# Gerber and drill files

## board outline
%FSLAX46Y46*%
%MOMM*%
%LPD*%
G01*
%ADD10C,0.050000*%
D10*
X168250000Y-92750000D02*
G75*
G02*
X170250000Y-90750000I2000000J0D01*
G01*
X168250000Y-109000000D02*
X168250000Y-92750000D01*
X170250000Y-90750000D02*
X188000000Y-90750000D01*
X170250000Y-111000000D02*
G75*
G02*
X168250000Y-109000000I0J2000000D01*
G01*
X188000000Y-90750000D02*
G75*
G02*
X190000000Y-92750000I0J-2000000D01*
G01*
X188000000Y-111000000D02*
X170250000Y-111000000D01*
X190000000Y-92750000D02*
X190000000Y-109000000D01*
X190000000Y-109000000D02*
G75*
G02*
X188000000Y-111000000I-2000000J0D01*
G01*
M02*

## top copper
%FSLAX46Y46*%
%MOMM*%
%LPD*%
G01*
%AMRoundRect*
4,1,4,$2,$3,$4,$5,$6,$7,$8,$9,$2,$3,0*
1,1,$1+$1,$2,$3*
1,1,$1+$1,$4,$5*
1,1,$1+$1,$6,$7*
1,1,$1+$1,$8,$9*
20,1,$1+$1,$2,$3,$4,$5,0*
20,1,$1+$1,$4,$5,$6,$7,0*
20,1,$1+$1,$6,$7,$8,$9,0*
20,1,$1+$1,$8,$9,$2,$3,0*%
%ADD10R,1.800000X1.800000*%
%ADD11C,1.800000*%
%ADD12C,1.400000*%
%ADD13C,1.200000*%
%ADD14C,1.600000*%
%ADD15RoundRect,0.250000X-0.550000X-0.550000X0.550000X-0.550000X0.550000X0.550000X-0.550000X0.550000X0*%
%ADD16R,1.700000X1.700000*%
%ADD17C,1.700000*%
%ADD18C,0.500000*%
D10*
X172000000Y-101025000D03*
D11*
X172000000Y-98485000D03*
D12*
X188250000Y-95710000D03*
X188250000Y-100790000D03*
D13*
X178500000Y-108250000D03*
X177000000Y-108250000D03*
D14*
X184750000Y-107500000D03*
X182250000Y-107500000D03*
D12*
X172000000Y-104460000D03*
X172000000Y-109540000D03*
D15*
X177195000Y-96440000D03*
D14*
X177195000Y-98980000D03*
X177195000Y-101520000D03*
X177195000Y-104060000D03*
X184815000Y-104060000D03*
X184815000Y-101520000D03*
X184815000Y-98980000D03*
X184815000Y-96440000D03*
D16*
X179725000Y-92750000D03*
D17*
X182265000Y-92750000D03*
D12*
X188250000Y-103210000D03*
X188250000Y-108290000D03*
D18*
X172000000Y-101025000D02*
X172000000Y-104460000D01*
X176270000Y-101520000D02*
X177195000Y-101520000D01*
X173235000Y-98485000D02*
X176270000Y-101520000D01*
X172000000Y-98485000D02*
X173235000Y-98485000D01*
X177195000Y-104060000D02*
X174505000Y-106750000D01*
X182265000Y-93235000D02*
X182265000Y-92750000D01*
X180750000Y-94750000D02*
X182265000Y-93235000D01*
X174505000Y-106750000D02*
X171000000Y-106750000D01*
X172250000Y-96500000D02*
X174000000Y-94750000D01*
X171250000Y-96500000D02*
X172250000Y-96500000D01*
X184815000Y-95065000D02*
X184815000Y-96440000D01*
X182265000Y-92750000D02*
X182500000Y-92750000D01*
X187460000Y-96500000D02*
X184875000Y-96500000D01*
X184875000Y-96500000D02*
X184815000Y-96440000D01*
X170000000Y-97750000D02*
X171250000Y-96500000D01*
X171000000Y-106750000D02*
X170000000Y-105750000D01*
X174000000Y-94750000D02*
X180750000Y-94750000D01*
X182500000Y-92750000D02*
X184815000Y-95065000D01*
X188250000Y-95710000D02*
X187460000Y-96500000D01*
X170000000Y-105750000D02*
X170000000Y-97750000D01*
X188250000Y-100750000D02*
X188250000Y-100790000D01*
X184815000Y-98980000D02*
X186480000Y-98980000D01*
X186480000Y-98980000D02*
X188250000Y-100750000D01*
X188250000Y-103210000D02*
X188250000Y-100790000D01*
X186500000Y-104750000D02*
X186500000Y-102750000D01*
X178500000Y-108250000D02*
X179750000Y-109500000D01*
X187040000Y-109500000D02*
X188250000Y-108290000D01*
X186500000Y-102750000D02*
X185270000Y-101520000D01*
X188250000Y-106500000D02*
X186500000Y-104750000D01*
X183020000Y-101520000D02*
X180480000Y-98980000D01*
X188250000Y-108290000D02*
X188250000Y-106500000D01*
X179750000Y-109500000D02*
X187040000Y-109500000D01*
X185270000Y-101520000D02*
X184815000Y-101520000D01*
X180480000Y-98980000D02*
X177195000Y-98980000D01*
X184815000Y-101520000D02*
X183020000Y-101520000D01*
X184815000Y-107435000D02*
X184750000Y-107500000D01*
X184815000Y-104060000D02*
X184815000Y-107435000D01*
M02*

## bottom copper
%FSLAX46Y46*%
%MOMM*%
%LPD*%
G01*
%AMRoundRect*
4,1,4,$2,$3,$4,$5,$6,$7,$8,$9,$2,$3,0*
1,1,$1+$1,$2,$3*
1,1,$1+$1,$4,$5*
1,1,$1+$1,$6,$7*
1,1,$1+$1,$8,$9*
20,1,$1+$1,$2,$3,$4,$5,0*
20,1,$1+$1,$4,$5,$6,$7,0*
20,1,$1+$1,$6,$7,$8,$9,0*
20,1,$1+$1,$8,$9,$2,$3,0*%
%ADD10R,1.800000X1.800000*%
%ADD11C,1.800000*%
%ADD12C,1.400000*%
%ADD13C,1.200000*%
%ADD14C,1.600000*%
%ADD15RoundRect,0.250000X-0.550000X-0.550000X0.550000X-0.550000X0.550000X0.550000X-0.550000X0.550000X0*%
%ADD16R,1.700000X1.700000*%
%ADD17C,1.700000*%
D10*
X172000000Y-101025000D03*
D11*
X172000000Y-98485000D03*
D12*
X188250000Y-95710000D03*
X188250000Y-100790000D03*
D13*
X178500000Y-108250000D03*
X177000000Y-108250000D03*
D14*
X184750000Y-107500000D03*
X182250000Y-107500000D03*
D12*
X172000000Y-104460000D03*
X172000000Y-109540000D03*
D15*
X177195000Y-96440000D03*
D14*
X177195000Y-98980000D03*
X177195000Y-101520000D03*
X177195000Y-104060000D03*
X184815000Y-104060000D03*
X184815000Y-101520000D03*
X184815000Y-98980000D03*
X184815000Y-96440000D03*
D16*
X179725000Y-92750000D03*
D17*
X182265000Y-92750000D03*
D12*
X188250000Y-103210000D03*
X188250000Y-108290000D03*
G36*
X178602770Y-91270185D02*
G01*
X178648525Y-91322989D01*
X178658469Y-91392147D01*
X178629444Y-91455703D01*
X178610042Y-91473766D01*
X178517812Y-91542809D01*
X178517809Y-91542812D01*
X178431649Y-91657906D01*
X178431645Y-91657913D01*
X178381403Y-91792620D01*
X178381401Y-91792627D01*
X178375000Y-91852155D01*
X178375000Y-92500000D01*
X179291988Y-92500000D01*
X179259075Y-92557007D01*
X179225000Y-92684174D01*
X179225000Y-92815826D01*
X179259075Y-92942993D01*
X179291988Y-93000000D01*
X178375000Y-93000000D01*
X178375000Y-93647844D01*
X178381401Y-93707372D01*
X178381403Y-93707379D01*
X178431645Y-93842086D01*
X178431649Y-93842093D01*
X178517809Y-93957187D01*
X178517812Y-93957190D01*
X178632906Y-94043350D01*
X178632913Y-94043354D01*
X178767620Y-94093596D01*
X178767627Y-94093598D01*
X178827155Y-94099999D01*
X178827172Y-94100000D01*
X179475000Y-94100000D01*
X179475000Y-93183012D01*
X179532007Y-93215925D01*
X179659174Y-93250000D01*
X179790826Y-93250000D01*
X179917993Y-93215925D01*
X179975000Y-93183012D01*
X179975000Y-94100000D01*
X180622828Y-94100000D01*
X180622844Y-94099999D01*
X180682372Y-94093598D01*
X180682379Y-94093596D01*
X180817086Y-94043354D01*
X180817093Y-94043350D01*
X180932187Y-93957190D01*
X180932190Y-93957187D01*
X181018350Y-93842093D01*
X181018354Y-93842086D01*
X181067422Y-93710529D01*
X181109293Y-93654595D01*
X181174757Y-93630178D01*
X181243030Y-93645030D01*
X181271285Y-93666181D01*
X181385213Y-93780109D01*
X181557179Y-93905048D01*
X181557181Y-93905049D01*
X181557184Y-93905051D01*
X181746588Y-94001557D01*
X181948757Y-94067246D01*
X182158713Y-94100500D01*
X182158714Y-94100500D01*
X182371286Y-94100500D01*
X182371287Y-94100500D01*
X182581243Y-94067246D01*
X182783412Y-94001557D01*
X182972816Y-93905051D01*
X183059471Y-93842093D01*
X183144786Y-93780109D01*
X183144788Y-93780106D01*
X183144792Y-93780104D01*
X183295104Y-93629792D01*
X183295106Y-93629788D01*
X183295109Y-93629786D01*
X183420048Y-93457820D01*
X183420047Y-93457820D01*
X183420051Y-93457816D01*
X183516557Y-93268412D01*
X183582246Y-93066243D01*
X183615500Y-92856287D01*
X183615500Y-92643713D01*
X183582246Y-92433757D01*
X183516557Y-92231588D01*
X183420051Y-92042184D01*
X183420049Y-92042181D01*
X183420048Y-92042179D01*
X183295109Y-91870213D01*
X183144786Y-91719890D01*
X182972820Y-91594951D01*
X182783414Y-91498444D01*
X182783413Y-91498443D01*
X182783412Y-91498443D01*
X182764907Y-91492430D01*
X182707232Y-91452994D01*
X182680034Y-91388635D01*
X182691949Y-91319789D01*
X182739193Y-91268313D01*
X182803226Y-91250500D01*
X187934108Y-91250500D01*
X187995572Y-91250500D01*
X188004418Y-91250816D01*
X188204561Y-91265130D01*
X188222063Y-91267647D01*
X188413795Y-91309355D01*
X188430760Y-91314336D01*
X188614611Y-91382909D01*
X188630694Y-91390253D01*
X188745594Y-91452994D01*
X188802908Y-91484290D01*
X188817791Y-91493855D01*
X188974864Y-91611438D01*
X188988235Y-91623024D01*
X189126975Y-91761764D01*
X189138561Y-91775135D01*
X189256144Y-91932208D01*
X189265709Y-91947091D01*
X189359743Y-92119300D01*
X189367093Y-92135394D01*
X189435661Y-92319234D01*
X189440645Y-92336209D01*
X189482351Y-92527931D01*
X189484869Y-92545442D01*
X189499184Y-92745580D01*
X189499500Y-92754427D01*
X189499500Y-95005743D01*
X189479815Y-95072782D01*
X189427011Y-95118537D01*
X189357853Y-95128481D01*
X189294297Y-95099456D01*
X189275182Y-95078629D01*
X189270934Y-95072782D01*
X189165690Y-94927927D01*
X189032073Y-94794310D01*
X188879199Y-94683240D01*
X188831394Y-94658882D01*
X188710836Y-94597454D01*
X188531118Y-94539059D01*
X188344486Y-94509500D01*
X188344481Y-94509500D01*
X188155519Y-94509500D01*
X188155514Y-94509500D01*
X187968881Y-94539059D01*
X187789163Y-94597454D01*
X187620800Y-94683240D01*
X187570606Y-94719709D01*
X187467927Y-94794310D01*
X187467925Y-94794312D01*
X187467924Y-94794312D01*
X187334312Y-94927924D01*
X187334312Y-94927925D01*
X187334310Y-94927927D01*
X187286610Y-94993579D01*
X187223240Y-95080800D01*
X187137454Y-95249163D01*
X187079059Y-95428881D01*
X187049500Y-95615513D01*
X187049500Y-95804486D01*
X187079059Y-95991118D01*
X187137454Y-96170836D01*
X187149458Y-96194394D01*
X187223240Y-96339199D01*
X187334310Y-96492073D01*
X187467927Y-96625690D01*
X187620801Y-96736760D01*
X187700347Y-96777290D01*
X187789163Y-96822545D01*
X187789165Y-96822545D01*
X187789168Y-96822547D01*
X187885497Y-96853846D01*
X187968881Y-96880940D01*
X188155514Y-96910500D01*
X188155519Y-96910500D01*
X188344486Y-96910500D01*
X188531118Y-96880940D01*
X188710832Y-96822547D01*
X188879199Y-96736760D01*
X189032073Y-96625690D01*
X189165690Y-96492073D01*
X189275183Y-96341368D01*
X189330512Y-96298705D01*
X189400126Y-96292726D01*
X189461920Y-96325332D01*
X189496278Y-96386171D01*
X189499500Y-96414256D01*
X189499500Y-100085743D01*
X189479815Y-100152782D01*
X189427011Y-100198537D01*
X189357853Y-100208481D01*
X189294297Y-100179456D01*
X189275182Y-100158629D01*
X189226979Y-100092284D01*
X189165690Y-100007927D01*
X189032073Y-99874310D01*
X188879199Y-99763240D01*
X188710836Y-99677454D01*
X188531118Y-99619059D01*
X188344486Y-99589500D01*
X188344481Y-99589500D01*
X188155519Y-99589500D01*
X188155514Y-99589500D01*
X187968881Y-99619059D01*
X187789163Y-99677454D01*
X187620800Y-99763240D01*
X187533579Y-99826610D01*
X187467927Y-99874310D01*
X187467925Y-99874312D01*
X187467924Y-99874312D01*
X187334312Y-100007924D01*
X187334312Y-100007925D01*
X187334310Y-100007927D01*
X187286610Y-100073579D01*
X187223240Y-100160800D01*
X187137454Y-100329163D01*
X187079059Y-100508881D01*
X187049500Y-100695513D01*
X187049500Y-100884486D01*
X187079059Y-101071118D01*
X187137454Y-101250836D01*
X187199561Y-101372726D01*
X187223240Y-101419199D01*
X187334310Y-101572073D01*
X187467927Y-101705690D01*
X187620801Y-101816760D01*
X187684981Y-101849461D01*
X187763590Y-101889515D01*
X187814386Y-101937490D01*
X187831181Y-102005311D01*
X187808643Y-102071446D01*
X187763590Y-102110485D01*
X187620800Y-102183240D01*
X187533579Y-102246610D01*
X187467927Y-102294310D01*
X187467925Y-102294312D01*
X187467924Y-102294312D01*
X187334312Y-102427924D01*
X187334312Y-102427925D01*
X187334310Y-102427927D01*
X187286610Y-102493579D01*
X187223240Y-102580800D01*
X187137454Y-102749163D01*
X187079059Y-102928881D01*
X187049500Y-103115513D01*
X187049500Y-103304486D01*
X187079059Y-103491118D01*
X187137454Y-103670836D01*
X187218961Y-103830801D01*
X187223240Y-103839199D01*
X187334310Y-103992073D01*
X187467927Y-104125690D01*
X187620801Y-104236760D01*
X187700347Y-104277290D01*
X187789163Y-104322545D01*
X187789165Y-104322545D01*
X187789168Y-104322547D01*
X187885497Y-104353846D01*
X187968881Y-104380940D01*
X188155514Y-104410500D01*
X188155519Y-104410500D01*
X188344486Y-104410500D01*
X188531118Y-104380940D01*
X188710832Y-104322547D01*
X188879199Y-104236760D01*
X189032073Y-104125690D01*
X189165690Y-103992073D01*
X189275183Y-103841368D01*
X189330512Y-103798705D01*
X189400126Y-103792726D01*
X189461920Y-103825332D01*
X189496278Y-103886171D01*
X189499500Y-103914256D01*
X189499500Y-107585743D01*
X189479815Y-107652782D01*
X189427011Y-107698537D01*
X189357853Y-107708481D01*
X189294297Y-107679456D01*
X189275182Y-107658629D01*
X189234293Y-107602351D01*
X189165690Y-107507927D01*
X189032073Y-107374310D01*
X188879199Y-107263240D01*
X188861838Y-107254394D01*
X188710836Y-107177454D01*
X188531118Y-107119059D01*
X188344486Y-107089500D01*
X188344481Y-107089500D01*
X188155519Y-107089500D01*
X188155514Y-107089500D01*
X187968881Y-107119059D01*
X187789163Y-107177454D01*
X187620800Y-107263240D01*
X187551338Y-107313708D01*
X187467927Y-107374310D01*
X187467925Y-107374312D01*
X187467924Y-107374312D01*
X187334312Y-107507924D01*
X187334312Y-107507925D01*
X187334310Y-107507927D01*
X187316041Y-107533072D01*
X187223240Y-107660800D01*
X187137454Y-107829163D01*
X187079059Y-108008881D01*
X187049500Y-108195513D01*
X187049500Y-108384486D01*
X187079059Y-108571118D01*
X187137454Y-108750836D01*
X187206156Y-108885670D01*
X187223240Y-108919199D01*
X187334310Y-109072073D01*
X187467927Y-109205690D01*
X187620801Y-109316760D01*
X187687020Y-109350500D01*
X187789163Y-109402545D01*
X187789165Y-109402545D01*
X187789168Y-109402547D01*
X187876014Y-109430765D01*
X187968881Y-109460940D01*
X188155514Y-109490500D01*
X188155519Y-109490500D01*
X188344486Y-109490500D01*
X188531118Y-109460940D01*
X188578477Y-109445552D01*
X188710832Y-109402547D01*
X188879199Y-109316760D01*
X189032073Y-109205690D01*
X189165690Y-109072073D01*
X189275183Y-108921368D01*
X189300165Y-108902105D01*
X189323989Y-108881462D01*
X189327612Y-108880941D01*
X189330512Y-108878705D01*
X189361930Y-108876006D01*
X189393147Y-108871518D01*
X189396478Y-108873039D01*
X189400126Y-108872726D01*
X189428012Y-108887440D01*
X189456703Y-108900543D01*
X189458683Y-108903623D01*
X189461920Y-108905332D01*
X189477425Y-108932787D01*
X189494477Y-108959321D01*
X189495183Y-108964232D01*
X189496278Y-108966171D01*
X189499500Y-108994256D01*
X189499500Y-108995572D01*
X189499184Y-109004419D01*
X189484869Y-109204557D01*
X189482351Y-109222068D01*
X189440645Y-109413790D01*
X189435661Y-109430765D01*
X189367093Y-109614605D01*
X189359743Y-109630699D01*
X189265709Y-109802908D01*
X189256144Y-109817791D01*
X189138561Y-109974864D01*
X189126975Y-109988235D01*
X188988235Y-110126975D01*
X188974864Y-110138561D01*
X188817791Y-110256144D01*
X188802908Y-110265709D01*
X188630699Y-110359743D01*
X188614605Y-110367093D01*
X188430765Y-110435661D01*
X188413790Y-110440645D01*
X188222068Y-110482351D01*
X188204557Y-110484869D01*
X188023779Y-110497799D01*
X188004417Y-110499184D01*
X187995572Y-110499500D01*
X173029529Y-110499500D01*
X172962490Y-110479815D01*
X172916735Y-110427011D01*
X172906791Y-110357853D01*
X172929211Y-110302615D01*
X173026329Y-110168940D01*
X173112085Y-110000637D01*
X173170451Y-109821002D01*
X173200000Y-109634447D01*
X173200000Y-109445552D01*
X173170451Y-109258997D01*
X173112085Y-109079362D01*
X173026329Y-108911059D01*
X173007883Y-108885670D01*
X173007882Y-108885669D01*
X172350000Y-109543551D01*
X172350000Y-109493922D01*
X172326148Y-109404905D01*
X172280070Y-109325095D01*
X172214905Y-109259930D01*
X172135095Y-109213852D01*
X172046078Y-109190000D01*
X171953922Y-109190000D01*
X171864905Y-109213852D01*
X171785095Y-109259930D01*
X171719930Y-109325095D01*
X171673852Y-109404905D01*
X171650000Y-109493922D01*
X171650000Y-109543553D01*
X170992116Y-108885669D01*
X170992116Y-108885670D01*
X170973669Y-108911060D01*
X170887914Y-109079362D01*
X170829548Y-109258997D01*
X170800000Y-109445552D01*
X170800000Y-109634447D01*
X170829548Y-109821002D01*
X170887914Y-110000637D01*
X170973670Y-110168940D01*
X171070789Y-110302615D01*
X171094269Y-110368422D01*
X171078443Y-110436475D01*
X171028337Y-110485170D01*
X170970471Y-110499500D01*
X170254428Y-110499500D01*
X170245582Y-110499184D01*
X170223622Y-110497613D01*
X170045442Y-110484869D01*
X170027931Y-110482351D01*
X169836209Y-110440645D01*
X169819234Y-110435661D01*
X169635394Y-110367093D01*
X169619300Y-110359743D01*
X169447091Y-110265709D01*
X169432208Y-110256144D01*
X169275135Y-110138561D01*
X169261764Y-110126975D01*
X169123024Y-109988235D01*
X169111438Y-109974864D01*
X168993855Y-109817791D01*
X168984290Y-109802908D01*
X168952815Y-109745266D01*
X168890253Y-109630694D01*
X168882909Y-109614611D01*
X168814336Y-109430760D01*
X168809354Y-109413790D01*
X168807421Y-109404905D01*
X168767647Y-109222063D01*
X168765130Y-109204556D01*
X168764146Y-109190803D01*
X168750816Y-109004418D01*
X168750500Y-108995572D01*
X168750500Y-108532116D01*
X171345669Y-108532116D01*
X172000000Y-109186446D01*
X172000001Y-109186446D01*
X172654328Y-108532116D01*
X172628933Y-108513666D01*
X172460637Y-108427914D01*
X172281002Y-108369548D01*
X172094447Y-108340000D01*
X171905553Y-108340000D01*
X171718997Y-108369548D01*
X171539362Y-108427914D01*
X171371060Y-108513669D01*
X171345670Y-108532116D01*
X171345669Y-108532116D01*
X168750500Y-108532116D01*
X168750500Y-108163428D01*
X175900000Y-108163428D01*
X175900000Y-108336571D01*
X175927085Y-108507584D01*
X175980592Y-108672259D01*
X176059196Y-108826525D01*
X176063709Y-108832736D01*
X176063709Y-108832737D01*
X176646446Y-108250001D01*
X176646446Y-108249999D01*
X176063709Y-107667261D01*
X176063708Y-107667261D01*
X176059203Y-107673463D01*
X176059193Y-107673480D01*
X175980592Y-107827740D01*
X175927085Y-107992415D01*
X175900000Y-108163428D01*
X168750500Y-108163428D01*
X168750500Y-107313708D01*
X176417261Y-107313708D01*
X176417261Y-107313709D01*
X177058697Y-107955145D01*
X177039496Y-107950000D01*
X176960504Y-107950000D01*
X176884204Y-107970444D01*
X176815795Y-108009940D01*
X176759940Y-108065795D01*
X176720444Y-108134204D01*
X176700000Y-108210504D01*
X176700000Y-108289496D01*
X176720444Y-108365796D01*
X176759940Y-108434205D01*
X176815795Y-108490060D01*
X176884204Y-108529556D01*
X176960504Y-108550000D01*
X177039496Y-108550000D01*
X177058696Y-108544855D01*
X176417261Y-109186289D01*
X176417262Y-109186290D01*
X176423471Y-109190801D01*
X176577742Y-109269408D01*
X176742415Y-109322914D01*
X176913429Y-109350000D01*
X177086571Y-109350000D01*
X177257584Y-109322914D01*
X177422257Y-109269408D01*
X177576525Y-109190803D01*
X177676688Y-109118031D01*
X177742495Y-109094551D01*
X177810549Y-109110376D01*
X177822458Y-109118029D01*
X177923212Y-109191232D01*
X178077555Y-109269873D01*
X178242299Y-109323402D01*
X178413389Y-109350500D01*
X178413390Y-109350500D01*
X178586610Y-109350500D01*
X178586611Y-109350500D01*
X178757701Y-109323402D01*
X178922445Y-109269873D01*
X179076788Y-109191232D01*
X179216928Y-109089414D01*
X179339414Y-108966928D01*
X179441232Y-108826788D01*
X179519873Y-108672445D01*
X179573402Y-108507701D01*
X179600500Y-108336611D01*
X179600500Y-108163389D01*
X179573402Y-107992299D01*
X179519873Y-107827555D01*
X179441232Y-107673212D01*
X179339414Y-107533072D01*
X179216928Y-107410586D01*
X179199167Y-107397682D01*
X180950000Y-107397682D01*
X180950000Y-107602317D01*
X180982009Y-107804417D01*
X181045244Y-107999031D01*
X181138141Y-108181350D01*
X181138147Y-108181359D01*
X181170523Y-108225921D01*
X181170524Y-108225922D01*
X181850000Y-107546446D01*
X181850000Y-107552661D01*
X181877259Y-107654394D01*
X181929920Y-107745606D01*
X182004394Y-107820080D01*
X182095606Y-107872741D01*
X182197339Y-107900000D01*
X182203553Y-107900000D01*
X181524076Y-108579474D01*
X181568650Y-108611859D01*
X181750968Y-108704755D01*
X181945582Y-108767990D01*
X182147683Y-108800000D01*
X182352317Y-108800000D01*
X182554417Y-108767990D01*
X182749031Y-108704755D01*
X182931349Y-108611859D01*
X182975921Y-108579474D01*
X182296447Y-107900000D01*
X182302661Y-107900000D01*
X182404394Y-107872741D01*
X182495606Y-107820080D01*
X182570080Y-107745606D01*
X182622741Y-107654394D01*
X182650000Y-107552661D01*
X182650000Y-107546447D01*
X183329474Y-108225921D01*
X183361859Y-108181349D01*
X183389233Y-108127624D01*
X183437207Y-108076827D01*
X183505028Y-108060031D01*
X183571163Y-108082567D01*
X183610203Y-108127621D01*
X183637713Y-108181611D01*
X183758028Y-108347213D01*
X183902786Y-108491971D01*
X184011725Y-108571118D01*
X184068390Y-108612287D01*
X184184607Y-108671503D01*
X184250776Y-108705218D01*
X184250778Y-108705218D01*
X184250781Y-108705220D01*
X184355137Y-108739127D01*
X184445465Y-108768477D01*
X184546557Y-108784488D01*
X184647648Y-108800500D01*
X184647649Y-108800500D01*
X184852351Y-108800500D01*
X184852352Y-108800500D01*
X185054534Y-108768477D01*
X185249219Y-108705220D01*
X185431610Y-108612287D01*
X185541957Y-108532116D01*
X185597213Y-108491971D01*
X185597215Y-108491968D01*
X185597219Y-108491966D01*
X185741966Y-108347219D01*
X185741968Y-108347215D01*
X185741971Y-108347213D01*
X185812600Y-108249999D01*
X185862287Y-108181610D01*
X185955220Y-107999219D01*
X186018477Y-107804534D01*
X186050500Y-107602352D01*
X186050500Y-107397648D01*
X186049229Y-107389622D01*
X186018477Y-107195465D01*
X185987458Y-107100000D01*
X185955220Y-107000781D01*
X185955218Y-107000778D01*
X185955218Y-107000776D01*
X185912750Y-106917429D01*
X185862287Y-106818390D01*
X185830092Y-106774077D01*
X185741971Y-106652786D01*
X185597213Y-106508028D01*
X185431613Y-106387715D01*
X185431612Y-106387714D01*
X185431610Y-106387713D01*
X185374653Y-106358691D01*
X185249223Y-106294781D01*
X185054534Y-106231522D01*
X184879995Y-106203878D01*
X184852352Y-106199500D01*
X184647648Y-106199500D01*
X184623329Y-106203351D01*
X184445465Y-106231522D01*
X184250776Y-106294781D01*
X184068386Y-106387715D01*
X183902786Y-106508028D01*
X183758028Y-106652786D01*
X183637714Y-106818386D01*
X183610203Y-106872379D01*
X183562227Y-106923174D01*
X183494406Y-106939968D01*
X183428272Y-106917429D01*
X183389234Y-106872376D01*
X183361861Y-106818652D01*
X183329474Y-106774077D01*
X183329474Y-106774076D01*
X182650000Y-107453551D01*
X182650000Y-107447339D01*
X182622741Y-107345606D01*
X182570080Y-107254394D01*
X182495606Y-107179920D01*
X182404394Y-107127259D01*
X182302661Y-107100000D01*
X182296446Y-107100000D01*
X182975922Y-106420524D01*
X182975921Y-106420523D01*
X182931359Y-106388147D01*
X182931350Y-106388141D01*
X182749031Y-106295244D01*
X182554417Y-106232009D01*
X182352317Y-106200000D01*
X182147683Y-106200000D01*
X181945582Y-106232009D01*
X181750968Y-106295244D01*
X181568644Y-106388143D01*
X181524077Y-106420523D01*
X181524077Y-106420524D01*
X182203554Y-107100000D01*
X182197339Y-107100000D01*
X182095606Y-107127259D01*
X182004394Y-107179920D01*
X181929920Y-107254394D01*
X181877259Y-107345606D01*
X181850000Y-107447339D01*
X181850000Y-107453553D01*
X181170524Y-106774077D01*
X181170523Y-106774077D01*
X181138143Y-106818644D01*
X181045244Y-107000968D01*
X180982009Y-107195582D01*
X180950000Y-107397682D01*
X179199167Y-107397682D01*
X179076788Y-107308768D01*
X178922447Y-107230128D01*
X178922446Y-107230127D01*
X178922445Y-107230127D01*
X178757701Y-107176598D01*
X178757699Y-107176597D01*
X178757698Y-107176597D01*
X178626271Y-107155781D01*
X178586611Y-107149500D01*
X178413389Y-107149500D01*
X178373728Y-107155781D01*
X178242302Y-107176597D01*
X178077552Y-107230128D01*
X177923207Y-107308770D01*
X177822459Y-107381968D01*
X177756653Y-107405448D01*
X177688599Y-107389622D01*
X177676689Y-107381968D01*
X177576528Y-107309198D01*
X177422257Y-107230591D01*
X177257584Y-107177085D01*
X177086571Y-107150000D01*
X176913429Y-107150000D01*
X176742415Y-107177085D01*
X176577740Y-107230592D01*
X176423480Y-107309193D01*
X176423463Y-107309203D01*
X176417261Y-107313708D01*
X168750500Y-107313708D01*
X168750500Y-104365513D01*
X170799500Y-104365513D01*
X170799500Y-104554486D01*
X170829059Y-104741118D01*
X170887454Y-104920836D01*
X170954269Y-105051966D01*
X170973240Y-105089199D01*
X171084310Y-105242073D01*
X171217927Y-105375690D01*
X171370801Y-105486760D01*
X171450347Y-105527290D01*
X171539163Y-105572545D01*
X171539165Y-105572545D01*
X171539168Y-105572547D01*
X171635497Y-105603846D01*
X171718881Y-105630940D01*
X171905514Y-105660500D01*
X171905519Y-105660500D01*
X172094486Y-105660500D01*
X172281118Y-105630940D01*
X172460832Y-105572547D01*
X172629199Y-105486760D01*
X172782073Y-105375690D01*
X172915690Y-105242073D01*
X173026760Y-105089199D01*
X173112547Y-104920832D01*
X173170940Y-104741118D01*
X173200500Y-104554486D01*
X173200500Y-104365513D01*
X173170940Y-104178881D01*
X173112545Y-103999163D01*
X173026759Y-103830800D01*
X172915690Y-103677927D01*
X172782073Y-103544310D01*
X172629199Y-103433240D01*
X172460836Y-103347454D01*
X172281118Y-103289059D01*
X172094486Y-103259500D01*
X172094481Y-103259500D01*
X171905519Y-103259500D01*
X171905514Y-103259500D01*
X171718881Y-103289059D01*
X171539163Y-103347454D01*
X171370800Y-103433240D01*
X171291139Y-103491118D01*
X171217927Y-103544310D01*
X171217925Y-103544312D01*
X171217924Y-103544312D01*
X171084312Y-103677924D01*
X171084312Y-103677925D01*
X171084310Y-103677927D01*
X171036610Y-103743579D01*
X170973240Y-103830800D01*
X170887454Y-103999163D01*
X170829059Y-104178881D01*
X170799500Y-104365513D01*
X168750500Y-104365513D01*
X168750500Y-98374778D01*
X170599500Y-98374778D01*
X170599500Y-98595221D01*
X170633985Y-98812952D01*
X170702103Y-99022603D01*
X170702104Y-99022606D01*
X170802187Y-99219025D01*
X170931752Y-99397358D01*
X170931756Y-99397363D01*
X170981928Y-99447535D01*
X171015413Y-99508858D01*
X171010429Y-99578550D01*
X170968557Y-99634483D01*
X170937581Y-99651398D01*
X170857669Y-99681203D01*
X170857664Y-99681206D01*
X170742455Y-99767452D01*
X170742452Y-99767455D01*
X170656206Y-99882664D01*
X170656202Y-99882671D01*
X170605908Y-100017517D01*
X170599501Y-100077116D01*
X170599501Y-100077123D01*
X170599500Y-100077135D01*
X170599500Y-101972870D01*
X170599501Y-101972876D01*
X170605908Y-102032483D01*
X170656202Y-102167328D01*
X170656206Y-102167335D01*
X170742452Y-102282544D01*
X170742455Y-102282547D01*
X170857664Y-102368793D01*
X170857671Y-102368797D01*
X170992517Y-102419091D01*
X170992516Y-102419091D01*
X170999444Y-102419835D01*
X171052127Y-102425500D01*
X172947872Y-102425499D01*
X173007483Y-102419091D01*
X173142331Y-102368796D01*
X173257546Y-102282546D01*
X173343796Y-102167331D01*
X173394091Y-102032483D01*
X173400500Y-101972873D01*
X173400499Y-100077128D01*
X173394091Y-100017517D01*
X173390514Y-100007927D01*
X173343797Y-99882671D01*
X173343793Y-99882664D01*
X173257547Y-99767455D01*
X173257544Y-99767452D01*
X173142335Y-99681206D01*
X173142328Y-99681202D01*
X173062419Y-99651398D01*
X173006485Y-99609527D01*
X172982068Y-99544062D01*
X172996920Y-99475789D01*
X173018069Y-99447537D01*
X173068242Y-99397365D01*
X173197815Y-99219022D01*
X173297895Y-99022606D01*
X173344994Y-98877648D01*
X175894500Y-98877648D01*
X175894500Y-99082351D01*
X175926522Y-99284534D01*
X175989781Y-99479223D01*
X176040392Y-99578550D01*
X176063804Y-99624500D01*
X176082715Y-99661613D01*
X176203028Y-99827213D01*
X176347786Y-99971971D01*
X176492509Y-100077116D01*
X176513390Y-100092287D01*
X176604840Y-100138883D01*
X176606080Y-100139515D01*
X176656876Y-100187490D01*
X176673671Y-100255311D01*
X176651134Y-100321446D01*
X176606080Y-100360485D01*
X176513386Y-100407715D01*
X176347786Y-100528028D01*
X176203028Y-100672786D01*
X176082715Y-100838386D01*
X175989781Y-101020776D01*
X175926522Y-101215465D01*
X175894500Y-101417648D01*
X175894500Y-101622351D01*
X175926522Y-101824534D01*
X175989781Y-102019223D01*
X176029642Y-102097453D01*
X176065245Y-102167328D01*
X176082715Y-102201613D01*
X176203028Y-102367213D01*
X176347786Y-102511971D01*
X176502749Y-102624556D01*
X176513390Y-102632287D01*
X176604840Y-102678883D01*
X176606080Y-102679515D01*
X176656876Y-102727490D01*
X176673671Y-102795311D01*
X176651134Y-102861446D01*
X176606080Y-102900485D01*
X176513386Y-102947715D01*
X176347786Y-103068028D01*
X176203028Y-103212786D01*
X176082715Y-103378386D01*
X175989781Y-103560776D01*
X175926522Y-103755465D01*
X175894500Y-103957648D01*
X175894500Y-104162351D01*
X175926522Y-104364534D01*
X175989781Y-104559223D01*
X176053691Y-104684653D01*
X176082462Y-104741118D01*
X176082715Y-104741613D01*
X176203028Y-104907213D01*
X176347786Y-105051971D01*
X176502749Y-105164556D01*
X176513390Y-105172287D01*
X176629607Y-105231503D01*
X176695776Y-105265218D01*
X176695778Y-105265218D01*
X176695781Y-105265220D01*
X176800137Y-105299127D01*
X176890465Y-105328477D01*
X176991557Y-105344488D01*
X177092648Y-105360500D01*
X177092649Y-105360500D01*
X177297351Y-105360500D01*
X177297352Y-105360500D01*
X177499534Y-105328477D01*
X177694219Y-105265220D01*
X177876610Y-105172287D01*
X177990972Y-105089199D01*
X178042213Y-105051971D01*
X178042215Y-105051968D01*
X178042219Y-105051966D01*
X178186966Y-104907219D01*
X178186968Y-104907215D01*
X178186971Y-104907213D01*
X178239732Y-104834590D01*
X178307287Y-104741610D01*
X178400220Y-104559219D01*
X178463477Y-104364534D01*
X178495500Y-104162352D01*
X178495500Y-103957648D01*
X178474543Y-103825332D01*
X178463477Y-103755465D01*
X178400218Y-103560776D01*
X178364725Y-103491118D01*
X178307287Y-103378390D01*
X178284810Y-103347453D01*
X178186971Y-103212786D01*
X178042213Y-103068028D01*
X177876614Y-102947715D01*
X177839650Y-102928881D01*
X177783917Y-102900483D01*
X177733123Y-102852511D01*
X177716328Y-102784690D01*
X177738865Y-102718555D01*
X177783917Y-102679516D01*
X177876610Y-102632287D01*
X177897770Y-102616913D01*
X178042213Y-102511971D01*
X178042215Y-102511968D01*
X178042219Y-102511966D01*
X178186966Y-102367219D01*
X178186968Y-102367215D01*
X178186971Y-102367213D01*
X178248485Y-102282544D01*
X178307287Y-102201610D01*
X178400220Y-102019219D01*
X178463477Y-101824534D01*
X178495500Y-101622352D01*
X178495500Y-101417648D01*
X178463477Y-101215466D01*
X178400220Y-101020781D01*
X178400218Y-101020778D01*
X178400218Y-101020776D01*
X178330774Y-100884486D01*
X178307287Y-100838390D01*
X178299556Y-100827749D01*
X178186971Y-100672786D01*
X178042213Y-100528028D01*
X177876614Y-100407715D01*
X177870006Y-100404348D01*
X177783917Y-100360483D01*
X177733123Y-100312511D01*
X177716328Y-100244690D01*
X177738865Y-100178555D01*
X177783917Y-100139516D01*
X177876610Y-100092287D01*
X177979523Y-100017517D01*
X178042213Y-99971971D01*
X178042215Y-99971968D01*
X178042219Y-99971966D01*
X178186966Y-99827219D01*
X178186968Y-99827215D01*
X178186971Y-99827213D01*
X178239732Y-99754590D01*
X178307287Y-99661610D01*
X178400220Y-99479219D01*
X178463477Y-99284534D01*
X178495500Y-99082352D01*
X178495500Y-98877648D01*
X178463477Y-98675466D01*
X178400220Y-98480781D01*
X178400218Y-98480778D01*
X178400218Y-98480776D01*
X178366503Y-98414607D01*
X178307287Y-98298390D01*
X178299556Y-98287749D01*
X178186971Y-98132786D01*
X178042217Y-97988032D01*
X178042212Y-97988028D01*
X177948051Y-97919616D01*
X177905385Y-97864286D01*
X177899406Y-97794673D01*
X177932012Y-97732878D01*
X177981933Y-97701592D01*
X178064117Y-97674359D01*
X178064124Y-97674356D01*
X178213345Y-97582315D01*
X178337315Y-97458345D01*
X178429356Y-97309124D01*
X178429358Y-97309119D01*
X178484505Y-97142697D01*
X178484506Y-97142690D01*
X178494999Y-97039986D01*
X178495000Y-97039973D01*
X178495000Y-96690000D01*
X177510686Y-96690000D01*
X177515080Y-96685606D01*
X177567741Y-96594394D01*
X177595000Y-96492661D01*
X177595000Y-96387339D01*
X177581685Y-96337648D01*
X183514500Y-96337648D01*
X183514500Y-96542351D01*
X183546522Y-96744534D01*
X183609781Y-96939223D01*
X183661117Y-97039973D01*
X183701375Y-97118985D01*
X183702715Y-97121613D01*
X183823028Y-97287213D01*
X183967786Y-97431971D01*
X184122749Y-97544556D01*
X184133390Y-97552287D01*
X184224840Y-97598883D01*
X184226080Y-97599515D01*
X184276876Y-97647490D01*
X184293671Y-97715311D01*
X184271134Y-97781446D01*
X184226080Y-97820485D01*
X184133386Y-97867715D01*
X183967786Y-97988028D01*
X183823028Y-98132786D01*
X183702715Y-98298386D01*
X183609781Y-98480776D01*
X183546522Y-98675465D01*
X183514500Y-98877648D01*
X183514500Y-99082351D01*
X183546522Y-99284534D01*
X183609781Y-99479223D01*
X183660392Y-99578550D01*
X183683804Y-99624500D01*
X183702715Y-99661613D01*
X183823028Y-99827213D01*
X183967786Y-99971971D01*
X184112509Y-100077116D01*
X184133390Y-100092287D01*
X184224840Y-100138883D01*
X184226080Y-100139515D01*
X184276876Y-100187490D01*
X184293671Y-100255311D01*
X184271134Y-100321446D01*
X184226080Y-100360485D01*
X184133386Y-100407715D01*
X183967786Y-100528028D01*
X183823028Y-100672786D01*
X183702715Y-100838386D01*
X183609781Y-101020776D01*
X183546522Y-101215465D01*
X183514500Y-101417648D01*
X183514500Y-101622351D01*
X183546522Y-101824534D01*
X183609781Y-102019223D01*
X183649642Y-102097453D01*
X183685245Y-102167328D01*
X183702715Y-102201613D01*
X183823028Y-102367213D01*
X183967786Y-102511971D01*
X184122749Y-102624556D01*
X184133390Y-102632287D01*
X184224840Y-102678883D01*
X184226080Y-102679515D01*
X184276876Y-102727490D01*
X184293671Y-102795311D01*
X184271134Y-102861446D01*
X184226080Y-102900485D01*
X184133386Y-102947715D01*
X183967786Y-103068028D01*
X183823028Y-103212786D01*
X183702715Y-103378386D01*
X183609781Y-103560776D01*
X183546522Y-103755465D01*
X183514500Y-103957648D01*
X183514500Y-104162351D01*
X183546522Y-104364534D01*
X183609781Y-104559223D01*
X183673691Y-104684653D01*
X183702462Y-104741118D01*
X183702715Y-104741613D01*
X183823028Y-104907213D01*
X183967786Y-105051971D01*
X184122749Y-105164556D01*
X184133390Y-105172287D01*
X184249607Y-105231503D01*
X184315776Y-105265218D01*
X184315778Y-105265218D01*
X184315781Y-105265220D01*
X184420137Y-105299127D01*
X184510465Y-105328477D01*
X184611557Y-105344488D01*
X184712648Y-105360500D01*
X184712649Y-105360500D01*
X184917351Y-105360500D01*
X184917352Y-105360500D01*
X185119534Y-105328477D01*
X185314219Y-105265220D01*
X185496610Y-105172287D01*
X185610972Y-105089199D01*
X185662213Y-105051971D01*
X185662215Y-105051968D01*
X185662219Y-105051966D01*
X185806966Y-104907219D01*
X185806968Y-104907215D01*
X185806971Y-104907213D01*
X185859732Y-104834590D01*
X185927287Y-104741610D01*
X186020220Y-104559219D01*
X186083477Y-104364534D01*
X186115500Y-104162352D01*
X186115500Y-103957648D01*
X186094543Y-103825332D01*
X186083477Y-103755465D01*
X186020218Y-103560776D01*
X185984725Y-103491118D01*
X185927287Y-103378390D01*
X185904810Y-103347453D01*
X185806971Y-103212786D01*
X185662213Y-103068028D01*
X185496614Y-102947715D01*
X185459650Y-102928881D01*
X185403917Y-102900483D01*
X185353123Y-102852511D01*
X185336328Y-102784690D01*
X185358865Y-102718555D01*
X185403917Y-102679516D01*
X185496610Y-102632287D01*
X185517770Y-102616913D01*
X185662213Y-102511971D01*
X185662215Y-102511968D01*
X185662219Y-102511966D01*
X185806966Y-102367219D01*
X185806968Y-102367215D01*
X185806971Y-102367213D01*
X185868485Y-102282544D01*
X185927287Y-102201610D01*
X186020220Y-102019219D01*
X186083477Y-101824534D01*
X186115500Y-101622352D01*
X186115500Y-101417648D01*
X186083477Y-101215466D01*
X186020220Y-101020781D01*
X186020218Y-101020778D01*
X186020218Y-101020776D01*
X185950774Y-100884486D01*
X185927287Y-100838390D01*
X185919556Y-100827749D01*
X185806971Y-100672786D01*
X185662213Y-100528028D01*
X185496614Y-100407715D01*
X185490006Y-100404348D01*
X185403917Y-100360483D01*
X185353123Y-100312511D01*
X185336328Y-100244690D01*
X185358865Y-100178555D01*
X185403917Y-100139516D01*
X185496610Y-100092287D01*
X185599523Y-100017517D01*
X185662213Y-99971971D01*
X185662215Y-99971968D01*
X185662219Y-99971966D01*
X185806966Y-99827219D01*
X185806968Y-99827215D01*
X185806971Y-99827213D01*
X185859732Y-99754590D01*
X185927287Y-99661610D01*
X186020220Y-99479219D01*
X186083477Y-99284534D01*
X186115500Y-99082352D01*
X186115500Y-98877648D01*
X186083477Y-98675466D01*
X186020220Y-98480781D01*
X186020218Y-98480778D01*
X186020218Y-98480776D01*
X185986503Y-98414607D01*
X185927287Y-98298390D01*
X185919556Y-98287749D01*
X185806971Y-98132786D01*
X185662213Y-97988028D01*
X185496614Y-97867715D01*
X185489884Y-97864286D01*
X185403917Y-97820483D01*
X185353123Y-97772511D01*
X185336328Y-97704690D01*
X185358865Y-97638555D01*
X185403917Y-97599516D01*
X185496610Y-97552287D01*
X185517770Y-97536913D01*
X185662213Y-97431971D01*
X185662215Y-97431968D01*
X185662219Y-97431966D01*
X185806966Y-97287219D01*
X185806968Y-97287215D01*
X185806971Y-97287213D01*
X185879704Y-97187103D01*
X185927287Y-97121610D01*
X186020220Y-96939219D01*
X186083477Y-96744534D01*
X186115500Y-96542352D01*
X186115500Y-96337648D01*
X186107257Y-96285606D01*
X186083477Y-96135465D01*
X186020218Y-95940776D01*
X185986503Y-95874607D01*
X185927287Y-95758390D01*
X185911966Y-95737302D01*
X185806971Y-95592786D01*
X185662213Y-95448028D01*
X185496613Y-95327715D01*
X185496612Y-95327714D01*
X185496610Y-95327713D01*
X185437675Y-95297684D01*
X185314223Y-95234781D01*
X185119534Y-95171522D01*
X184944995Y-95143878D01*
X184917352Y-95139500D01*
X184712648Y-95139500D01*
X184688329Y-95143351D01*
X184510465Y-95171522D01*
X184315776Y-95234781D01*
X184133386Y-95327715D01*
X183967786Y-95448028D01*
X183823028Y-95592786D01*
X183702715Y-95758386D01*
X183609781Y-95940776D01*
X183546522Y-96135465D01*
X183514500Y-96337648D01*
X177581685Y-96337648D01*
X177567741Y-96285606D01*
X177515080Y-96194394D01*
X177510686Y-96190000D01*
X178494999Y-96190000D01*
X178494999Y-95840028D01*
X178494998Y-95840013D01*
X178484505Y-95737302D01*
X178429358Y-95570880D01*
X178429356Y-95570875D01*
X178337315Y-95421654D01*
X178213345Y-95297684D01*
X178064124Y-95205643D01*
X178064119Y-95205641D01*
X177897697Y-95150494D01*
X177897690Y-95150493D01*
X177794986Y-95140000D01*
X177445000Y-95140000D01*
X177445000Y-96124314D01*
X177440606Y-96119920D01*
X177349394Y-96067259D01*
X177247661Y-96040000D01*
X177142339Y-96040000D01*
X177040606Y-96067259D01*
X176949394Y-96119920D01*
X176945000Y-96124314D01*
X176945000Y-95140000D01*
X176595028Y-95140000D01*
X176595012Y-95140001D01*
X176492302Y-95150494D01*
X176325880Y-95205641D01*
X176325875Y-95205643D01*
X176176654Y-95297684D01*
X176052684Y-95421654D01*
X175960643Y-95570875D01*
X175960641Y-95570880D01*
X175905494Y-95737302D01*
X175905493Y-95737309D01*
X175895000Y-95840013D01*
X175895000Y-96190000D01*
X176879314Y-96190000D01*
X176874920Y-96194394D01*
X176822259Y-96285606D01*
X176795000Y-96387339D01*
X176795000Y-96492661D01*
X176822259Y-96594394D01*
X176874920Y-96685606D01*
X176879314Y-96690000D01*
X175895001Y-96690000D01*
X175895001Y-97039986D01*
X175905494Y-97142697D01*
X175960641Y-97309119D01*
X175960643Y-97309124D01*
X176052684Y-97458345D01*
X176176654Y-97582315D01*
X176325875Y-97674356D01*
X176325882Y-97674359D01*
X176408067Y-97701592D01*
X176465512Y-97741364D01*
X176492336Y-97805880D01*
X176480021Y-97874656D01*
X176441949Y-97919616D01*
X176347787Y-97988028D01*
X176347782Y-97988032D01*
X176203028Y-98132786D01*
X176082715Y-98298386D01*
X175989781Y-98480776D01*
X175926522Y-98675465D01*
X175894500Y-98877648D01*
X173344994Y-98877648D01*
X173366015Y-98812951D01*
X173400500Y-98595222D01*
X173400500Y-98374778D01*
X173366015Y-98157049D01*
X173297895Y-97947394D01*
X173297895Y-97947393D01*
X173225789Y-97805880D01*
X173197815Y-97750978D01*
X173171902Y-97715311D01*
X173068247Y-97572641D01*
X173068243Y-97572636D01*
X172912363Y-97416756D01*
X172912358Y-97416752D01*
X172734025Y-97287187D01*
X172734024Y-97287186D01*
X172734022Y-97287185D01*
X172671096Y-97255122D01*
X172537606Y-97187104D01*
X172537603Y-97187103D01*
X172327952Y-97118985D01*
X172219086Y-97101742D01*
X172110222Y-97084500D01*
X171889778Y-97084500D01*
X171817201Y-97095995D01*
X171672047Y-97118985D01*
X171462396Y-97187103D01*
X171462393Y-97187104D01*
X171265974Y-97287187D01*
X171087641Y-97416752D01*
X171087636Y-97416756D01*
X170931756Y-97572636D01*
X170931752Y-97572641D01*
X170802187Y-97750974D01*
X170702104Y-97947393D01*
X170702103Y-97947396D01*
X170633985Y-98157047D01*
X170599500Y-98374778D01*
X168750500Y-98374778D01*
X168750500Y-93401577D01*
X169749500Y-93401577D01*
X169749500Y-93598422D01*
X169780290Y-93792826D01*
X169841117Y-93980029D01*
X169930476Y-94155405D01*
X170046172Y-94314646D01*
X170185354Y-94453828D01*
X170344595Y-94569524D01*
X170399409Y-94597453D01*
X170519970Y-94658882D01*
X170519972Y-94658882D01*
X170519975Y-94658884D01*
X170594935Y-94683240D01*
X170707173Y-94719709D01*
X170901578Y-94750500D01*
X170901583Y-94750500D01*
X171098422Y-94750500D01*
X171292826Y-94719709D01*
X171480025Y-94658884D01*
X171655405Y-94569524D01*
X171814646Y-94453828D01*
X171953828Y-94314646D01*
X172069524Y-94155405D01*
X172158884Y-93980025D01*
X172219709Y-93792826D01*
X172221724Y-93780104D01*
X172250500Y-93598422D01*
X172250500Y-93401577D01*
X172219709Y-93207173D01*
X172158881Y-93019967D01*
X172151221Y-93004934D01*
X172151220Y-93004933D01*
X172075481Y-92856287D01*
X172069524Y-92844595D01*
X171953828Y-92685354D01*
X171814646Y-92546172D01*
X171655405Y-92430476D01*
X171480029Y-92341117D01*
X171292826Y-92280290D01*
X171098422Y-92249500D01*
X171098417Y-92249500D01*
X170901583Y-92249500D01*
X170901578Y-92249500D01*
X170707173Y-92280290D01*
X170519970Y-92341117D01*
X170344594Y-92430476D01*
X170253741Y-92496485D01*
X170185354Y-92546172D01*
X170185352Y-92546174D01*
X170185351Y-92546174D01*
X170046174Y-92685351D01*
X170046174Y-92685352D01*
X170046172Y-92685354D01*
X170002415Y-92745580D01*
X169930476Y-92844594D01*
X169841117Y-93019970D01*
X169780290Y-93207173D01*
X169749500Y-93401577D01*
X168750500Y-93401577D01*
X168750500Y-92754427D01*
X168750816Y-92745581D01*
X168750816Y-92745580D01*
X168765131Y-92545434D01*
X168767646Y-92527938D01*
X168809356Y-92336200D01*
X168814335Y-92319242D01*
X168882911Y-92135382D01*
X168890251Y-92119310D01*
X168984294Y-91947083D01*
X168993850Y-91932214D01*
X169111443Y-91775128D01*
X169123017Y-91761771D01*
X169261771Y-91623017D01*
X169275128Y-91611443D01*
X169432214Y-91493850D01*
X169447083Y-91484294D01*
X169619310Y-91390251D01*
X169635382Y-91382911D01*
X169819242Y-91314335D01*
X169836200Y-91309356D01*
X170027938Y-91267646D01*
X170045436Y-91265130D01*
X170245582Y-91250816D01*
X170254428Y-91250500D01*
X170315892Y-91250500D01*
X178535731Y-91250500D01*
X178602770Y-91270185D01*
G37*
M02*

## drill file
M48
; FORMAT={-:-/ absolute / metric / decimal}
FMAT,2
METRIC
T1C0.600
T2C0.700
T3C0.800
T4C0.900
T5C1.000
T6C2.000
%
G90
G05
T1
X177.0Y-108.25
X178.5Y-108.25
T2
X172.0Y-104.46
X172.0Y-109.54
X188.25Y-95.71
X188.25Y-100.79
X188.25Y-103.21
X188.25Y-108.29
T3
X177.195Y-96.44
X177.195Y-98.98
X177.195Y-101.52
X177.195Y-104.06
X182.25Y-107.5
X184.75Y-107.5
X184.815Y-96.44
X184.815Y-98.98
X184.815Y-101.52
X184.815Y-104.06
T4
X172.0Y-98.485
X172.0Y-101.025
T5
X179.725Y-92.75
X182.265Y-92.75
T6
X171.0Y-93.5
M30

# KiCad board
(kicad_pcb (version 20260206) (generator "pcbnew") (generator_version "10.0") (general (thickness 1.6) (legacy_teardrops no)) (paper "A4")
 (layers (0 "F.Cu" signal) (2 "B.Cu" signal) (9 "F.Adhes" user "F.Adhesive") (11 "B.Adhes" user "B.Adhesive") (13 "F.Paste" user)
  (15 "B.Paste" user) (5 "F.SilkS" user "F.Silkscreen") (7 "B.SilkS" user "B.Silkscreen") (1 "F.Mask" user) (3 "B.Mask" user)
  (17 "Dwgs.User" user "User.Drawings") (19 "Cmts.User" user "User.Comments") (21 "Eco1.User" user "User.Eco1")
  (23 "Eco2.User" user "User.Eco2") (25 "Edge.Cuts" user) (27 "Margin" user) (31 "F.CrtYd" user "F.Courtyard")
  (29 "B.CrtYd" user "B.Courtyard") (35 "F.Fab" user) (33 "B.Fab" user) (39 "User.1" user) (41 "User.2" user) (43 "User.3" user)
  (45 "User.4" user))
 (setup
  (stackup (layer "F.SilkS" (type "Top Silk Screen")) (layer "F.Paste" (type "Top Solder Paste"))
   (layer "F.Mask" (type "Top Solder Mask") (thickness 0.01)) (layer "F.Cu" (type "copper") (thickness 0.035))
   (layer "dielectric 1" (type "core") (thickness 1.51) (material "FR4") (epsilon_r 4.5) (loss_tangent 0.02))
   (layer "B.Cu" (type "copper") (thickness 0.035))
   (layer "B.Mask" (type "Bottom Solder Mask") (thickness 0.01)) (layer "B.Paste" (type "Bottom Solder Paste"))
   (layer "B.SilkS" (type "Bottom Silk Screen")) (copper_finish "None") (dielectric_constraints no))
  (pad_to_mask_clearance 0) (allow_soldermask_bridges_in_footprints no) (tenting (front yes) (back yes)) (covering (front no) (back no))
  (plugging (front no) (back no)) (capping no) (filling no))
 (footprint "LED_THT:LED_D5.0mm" (layer "F.Cu") (at 172 101.025 90)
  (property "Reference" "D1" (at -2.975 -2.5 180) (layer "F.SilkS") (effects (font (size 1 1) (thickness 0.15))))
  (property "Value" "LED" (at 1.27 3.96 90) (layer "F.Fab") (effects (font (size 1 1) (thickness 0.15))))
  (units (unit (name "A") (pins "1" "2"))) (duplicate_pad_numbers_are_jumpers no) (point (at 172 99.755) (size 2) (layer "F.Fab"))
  (pad "1" thru_hole rect (at 0 0 90) (size 1.8 1.8) (drill 0.9) (layers "*.Cu" "*.Mask") (remove_unused_layers no) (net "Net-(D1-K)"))
  (pad "2" thru_hole circle (at 2.54 0 90) (size 1.8 1.8) (drill 0.9) (layers "*.Cu" "*.Mask") (remove_unused_layers no) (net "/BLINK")))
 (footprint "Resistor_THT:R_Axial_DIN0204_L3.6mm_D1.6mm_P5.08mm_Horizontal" (layer "F.Cu") (at 188.25 95.71 -90)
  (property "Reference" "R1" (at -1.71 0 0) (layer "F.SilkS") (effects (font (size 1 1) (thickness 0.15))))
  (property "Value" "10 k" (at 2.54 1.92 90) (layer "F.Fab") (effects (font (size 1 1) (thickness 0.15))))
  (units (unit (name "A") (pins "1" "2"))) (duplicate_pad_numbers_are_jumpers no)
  (pad "1" thru_hole circle (at 0 0 270) (size 1.4 1.4) (drill 0.7) (layers "*.Cu" "*.Mask") (remove_unused_layers no) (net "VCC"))
  (pad "2" thru_hole circle (at 5.08 0 270) (size 1.4 1.4) (drill 0.7) (layers "*.Cu" "*.Mask") (remove_unused_layers no) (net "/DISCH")))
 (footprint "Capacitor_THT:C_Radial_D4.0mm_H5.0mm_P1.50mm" (layer "F.Cu") (at 178.5 108.25 180)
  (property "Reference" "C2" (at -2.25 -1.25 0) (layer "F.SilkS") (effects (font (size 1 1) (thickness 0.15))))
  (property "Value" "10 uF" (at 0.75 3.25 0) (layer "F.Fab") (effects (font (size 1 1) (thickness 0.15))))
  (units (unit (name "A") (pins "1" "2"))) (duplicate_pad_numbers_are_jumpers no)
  (pad "1" thru_hole circle (at 0 0 180) (size 1.2 1.2) (drill 0.6) (layers "*.Cu" "*.Mask") (remove_unused_layers no) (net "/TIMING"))
  (pad "2" thru_hole circle (at 1.5 0 180) (size 1.2 1.2) (drill 0.6) (layers "*.Cu" "*.Mask") (remove_unused_layers no) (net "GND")))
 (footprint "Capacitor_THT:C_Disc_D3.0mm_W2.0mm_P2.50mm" (layer "F.Cu") (at 184.75 107.5 180)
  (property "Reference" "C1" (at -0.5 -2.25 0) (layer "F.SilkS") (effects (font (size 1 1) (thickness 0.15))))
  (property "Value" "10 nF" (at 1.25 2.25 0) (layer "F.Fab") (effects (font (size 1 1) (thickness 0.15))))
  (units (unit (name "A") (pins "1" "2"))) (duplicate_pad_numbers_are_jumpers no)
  (pad "1" thru_hole circle (at 0 0 180) (size 1.6 1.6) (drill 0.8) (layers "*.Cu" "*.Mask") (remove_unused_layers no) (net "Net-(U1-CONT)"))
  (pad "2" thru_hole circle (at 2.5 0 180) (size 1.6 1.6) (drill 0.8) (layers "*.Cu" "*.Mask") (remove_unused_layers no) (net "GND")))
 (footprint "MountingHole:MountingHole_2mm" (layer "F.Cu") (at 171 93.5)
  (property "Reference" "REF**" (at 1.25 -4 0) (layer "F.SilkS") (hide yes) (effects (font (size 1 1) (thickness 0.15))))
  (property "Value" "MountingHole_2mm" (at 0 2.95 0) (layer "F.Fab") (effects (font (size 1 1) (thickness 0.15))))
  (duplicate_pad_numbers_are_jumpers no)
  (pad "" np_thru_hole circle (at 0 0) (size 2 2) (drill 2) (layers "*.Cu" "*.Mask")))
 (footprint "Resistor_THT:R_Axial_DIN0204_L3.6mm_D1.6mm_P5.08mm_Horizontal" (layer "F.Cu") (at 172 104.46 -90)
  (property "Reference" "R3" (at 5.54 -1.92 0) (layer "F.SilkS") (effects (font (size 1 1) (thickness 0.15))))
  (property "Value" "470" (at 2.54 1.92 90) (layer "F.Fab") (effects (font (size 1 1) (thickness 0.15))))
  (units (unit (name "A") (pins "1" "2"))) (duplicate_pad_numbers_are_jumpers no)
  (pad "1" thru_hole circle (at 0 0 270) (size 1.4 1.4) (drill 0.7) (layers "*.Cu" "*.Mask") (remove_unused_layers no) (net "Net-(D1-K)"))
  (pad "2" thru_hole circle (at 5.08 0 270) (size 1.4 1.4) (drill 0.7) (layers "*.Cu" "*.Mask") (remove_unused_layers no) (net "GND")))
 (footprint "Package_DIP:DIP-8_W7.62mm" (layer "F.Cu") (at 177.195 96.44)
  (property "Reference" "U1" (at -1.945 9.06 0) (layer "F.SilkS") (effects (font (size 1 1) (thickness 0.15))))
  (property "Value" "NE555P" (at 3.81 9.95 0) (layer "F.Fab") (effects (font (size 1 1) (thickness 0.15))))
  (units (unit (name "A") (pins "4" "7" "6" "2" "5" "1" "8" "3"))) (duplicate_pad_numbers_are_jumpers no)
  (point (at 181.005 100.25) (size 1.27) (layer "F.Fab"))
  (pad "1" thru_hole roundrect (at 0 0) (size 1.6 1.6) (drill 0.8) (layers "*.Cu" "*.Mask") (remove_unused_layers no)
   (roundrect_rratio 0.15625) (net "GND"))
  (pad "2" thru_hole circle (at 0 2.54) (size 1.6 1.6) (drill 0.8) (layers "*.Cu" "*.Mask") (remove_unused_layers no) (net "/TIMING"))
  (pad "3" thru_hole circle (at 0 5.08) (size 1.6 1.6) (drill 0.8) (layers "*.Cu" "*.Mask") (remove_unused_layers no) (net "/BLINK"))
  (pad "4" thru_hole circle (at 0 7.62) (size 1.6 1.6) (drill 0.8) (layers "*.Cu" "*.Mask") (remove_unused_layers no) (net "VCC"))
  (pad "5" thru_hole circle (at 7.62 7.62) (size 1.6 1.6) (drill 0.8) (layers "*.Cu" "*.Mask") (remove_unused_layers no)
   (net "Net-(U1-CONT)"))
  (pad "6" thru_hole circle (at 7.62 5.08) (size 1.6 1.6) (drill 0.8) (layers "*.Cu" "*.Mask") (remove_unused_layers no) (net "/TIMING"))
  (pad "7" thru_hole circle (at 7.62 2.54) (size 1.6 1.6) (drill 0.8) (layers "*.Cu" "*.Mask") (remove_unused_layers no) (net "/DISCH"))
  (pad "8" thru_hole circle (at 7.62 0) (size 1.6 1.6) (drill 0.8) (layers "*.Cu" "*.Mask") (remove_unused_layers no) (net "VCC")))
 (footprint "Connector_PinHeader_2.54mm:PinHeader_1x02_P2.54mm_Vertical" (layer "F.Cu") (at 179.725 92.75 90)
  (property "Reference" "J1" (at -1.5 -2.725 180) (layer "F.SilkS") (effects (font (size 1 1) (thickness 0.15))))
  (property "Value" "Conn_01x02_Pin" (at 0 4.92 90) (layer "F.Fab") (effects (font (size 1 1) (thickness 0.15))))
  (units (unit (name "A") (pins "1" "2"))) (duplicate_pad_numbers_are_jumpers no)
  (pad "1" thru_hole rect (at 0 0 90) (size 1.7 1.7) (drill 1) (layers "*.Cu" "*.Mask") (remove_unused_layers no) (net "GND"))
  (pad "2" thru_hole circle (at 0 2.54 90) (size 1.7 1.7) (drill 1) (layers "*.Cu" "*.Mask") (remove_unused_layers no) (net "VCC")))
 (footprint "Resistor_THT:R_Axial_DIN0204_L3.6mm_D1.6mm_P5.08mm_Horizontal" (layer "F.Cu") (at 188.25 103.21 -90)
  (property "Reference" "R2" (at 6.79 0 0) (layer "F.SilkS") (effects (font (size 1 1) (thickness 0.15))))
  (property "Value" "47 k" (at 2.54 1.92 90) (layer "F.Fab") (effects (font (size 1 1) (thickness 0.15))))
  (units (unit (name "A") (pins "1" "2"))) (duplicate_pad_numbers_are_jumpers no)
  (pad "1" thru_hole circle (at 0 0 270) (size 1.4 1.4) (drill 0.7) (layers "*.Cu" "*.Mask") (remove_unused_layers no) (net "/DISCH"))
  (pad "2" thru_hole circle (at 5.08 0 270) (size 1.4 1.4) (drill 0.7) (layers "*.Cu" "*.Mask") (remove_unused_layers no) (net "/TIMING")))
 (gr_arc (start 168.25 92.75) (mid 168.835786 91.335786) (end 170.25 90.75) (stroke (width 0.05) (type default)) (layer "Edge.Cuts"))
 (gr_line (start 168.25 109) (end 168.25 92.75) (stroke (width 0.05) (type default)) (layer "Edge.Cuts"))
 (gr_line (start 170.25 90.75) (end 188 90.75) (stroke (width 0.05) (type default)) (layer "Edge.Cuts"))
 (gr_arc (start 170.25 111) (mid 168.835786 110.414214) (end 168.25 109) (stroke (width 0.05) (type default)) (layer "Edge.Cuts"))
 (gr_arc (start 188 90.75) (mid 189.414214 91.335786) (end 190 92.75) (stroke (width 0.05) (type default)) (layer "Edge.Cuts"))
 (gr_line (start 188 111) (end 170.25 111) (stroke (width 0.05) (type default)) (layer "Edge.Cuts"))
 (gr_line (start 190 92.75) (end 190 109) (stroke (width 0.05) (type default)) (layer "Edge.Cuts"))
 (gr_arc (start 190 109) (mid 189.414214 110.414214) (end 188 111) (stroke (width 0.05) (type default)) (layer "Edge.Cuts"))
 (segment (start 172 101.025) (end 172 104.46) (width 0.5) (layer "F.Cu") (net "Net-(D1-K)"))
 (segment (start 176.27 101.52) (end 177.195 101.52) (width 0.5) (layer "F.Cu") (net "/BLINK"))
 (segment (start 173.235 98.485) (end 176.27 101.52) (width 0.5) (layer "F.Cu") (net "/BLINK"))
 (segment (start 172 98.485) (end 173.235 98.485) (width 0.5) (layer "F.Cu") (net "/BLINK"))
 (segment (start 177.195 104.06) (end 174.505 106.75) (width 0.5) (layer "F.Cu") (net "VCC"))
 (segment (start 182.265 93.235) (end 182.265 92.75) (width 0.5) (layer "F.Cu") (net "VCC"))
 (segment (start 180.75 94.75) (end 182.265 93.235) (width 0.5) (layer "F.Cu") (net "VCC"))
 (segment (start 174.505 106.75) (end 171 106.75) (width 0.5) (layer "F.Cu") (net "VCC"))
 (segment (start 172.25 96.5) (end 174 94.75) (width 0.5) (layer "F.Cu") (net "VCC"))
 (segment (start 171.25 96.5) (end 172.25 96.5) (width 0.5) (layer "F.Cu") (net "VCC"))
 (segment (start 184.815 95.065) (end 184.815 96.44) (width 0.5) (layer "F.Cu") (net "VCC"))
 (segment (start 182.265 92.75) (end 182.5 92.75) (width 0.5) (layer "F.Cu") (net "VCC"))
 (segment (start 187.46 96.5) (end 184.875 96.5) (width 0.5) (layer "F.Cu") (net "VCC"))
 (segment (start 184.875 96.5) (end 184.815 96.44) (width 0.5) (layer "F.Cu") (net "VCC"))
 (segment (start 170 97.75) (end 171.25 96.5) (width 0.5) (layer "F.Cu") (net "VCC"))
 (segment (start 171 106.75) (end 170 105.75) (width 0.5) (layer "F.Cu") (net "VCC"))
 (segment (start 174 94.75) (end 180.75 94.75) (width 0.5) (layer "F.Cu") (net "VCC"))
 (segment (start 182.5 92.75) (end 184.815 95.065) (width 0.5) (layer "F.Cu") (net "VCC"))
 (segment (start 188.25 95.71) (end 187.46 96.5) (width 0.5) (layer "F.Cu") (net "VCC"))
 (segment (start 170 105.75) (end 170 97.75) (width 0.5) (layer "F.Cu") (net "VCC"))
 (segment (start 188.25 100.75) (end 188.25 100.79) (width 0.5) (layer "F.Cu") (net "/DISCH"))
 (segment (start 184.815 98.98) (end 186.48 98.98) (width 0.5) (layer "F.Cu") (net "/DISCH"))
 (segment (start 186.48 98.98) (end 188.25 100.75) (width 0.5) (layer "F.Cu") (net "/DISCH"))
 (segment (start 188.25 103.21) (end 188.25 100.79) (width 0.5) (layer "F.Cu") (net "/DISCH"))
 (segment (start 186.5 104.75) (end 186.5 102.75) (width 0.5) (layer "F.Cu") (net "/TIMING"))
 (segment (start 178.5 108.25) (end 179.75 109.5) (width 0.5) (layer "F.Cu") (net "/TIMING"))
 (segment (start 187.04 109.5) (end 188.25 108.29) (width 0.5) (layer "F.Cu") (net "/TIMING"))
 (segment (start 186.5 102.75) (end 185.27 101.52) (width 0.5) (layer "F.Cu") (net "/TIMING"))
 (segment (start 188.25 106.5) (end 186.5 104.75) (width 0.5) (layer "F.Cu") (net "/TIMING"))
 (segment (start 183.02 101.52) (end 180.48 98.98) (width 0.5) (layer "F.Cu") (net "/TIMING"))
 (segment (start 188.25 108.29) (end 188.25 106.5) (width 0.5) (layer "F.Cu") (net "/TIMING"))
 (segment (start 179.75 109.5) (end 187.04 109.5) (width 0.5) (layer "F.Cu") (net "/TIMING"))
 (segment (start 185.27 101.52) (end 184.815 101.52) (width 0.5) (layer "F.Cu") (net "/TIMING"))
 (segment (start 180.48 98.98) (end 177.195 98.98) (width 0.5) (layer "F.Cu") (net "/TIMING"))
 (segment (start 184.815 101.52) (end 183.02 101.52) (width 0.5) (layer "F.Cu") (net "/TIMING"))
 (segment (start 184.815 107.435) (end 184.75 107.5) (width 0.5) (layer "F.Cu") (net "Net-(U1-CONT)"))
 (segment (start 184.815 104.06) (end 184.815 107.435) (width 0.5) (layer "F.Cu") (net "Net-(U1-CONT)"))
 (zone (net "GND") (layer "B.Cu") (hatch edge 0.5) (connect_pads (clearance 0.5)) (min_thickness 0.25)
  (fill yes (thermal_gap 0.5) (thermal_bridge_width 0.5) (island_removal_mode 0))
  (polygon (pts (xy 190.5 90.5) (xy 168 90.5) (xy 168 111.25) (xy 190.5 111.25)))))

